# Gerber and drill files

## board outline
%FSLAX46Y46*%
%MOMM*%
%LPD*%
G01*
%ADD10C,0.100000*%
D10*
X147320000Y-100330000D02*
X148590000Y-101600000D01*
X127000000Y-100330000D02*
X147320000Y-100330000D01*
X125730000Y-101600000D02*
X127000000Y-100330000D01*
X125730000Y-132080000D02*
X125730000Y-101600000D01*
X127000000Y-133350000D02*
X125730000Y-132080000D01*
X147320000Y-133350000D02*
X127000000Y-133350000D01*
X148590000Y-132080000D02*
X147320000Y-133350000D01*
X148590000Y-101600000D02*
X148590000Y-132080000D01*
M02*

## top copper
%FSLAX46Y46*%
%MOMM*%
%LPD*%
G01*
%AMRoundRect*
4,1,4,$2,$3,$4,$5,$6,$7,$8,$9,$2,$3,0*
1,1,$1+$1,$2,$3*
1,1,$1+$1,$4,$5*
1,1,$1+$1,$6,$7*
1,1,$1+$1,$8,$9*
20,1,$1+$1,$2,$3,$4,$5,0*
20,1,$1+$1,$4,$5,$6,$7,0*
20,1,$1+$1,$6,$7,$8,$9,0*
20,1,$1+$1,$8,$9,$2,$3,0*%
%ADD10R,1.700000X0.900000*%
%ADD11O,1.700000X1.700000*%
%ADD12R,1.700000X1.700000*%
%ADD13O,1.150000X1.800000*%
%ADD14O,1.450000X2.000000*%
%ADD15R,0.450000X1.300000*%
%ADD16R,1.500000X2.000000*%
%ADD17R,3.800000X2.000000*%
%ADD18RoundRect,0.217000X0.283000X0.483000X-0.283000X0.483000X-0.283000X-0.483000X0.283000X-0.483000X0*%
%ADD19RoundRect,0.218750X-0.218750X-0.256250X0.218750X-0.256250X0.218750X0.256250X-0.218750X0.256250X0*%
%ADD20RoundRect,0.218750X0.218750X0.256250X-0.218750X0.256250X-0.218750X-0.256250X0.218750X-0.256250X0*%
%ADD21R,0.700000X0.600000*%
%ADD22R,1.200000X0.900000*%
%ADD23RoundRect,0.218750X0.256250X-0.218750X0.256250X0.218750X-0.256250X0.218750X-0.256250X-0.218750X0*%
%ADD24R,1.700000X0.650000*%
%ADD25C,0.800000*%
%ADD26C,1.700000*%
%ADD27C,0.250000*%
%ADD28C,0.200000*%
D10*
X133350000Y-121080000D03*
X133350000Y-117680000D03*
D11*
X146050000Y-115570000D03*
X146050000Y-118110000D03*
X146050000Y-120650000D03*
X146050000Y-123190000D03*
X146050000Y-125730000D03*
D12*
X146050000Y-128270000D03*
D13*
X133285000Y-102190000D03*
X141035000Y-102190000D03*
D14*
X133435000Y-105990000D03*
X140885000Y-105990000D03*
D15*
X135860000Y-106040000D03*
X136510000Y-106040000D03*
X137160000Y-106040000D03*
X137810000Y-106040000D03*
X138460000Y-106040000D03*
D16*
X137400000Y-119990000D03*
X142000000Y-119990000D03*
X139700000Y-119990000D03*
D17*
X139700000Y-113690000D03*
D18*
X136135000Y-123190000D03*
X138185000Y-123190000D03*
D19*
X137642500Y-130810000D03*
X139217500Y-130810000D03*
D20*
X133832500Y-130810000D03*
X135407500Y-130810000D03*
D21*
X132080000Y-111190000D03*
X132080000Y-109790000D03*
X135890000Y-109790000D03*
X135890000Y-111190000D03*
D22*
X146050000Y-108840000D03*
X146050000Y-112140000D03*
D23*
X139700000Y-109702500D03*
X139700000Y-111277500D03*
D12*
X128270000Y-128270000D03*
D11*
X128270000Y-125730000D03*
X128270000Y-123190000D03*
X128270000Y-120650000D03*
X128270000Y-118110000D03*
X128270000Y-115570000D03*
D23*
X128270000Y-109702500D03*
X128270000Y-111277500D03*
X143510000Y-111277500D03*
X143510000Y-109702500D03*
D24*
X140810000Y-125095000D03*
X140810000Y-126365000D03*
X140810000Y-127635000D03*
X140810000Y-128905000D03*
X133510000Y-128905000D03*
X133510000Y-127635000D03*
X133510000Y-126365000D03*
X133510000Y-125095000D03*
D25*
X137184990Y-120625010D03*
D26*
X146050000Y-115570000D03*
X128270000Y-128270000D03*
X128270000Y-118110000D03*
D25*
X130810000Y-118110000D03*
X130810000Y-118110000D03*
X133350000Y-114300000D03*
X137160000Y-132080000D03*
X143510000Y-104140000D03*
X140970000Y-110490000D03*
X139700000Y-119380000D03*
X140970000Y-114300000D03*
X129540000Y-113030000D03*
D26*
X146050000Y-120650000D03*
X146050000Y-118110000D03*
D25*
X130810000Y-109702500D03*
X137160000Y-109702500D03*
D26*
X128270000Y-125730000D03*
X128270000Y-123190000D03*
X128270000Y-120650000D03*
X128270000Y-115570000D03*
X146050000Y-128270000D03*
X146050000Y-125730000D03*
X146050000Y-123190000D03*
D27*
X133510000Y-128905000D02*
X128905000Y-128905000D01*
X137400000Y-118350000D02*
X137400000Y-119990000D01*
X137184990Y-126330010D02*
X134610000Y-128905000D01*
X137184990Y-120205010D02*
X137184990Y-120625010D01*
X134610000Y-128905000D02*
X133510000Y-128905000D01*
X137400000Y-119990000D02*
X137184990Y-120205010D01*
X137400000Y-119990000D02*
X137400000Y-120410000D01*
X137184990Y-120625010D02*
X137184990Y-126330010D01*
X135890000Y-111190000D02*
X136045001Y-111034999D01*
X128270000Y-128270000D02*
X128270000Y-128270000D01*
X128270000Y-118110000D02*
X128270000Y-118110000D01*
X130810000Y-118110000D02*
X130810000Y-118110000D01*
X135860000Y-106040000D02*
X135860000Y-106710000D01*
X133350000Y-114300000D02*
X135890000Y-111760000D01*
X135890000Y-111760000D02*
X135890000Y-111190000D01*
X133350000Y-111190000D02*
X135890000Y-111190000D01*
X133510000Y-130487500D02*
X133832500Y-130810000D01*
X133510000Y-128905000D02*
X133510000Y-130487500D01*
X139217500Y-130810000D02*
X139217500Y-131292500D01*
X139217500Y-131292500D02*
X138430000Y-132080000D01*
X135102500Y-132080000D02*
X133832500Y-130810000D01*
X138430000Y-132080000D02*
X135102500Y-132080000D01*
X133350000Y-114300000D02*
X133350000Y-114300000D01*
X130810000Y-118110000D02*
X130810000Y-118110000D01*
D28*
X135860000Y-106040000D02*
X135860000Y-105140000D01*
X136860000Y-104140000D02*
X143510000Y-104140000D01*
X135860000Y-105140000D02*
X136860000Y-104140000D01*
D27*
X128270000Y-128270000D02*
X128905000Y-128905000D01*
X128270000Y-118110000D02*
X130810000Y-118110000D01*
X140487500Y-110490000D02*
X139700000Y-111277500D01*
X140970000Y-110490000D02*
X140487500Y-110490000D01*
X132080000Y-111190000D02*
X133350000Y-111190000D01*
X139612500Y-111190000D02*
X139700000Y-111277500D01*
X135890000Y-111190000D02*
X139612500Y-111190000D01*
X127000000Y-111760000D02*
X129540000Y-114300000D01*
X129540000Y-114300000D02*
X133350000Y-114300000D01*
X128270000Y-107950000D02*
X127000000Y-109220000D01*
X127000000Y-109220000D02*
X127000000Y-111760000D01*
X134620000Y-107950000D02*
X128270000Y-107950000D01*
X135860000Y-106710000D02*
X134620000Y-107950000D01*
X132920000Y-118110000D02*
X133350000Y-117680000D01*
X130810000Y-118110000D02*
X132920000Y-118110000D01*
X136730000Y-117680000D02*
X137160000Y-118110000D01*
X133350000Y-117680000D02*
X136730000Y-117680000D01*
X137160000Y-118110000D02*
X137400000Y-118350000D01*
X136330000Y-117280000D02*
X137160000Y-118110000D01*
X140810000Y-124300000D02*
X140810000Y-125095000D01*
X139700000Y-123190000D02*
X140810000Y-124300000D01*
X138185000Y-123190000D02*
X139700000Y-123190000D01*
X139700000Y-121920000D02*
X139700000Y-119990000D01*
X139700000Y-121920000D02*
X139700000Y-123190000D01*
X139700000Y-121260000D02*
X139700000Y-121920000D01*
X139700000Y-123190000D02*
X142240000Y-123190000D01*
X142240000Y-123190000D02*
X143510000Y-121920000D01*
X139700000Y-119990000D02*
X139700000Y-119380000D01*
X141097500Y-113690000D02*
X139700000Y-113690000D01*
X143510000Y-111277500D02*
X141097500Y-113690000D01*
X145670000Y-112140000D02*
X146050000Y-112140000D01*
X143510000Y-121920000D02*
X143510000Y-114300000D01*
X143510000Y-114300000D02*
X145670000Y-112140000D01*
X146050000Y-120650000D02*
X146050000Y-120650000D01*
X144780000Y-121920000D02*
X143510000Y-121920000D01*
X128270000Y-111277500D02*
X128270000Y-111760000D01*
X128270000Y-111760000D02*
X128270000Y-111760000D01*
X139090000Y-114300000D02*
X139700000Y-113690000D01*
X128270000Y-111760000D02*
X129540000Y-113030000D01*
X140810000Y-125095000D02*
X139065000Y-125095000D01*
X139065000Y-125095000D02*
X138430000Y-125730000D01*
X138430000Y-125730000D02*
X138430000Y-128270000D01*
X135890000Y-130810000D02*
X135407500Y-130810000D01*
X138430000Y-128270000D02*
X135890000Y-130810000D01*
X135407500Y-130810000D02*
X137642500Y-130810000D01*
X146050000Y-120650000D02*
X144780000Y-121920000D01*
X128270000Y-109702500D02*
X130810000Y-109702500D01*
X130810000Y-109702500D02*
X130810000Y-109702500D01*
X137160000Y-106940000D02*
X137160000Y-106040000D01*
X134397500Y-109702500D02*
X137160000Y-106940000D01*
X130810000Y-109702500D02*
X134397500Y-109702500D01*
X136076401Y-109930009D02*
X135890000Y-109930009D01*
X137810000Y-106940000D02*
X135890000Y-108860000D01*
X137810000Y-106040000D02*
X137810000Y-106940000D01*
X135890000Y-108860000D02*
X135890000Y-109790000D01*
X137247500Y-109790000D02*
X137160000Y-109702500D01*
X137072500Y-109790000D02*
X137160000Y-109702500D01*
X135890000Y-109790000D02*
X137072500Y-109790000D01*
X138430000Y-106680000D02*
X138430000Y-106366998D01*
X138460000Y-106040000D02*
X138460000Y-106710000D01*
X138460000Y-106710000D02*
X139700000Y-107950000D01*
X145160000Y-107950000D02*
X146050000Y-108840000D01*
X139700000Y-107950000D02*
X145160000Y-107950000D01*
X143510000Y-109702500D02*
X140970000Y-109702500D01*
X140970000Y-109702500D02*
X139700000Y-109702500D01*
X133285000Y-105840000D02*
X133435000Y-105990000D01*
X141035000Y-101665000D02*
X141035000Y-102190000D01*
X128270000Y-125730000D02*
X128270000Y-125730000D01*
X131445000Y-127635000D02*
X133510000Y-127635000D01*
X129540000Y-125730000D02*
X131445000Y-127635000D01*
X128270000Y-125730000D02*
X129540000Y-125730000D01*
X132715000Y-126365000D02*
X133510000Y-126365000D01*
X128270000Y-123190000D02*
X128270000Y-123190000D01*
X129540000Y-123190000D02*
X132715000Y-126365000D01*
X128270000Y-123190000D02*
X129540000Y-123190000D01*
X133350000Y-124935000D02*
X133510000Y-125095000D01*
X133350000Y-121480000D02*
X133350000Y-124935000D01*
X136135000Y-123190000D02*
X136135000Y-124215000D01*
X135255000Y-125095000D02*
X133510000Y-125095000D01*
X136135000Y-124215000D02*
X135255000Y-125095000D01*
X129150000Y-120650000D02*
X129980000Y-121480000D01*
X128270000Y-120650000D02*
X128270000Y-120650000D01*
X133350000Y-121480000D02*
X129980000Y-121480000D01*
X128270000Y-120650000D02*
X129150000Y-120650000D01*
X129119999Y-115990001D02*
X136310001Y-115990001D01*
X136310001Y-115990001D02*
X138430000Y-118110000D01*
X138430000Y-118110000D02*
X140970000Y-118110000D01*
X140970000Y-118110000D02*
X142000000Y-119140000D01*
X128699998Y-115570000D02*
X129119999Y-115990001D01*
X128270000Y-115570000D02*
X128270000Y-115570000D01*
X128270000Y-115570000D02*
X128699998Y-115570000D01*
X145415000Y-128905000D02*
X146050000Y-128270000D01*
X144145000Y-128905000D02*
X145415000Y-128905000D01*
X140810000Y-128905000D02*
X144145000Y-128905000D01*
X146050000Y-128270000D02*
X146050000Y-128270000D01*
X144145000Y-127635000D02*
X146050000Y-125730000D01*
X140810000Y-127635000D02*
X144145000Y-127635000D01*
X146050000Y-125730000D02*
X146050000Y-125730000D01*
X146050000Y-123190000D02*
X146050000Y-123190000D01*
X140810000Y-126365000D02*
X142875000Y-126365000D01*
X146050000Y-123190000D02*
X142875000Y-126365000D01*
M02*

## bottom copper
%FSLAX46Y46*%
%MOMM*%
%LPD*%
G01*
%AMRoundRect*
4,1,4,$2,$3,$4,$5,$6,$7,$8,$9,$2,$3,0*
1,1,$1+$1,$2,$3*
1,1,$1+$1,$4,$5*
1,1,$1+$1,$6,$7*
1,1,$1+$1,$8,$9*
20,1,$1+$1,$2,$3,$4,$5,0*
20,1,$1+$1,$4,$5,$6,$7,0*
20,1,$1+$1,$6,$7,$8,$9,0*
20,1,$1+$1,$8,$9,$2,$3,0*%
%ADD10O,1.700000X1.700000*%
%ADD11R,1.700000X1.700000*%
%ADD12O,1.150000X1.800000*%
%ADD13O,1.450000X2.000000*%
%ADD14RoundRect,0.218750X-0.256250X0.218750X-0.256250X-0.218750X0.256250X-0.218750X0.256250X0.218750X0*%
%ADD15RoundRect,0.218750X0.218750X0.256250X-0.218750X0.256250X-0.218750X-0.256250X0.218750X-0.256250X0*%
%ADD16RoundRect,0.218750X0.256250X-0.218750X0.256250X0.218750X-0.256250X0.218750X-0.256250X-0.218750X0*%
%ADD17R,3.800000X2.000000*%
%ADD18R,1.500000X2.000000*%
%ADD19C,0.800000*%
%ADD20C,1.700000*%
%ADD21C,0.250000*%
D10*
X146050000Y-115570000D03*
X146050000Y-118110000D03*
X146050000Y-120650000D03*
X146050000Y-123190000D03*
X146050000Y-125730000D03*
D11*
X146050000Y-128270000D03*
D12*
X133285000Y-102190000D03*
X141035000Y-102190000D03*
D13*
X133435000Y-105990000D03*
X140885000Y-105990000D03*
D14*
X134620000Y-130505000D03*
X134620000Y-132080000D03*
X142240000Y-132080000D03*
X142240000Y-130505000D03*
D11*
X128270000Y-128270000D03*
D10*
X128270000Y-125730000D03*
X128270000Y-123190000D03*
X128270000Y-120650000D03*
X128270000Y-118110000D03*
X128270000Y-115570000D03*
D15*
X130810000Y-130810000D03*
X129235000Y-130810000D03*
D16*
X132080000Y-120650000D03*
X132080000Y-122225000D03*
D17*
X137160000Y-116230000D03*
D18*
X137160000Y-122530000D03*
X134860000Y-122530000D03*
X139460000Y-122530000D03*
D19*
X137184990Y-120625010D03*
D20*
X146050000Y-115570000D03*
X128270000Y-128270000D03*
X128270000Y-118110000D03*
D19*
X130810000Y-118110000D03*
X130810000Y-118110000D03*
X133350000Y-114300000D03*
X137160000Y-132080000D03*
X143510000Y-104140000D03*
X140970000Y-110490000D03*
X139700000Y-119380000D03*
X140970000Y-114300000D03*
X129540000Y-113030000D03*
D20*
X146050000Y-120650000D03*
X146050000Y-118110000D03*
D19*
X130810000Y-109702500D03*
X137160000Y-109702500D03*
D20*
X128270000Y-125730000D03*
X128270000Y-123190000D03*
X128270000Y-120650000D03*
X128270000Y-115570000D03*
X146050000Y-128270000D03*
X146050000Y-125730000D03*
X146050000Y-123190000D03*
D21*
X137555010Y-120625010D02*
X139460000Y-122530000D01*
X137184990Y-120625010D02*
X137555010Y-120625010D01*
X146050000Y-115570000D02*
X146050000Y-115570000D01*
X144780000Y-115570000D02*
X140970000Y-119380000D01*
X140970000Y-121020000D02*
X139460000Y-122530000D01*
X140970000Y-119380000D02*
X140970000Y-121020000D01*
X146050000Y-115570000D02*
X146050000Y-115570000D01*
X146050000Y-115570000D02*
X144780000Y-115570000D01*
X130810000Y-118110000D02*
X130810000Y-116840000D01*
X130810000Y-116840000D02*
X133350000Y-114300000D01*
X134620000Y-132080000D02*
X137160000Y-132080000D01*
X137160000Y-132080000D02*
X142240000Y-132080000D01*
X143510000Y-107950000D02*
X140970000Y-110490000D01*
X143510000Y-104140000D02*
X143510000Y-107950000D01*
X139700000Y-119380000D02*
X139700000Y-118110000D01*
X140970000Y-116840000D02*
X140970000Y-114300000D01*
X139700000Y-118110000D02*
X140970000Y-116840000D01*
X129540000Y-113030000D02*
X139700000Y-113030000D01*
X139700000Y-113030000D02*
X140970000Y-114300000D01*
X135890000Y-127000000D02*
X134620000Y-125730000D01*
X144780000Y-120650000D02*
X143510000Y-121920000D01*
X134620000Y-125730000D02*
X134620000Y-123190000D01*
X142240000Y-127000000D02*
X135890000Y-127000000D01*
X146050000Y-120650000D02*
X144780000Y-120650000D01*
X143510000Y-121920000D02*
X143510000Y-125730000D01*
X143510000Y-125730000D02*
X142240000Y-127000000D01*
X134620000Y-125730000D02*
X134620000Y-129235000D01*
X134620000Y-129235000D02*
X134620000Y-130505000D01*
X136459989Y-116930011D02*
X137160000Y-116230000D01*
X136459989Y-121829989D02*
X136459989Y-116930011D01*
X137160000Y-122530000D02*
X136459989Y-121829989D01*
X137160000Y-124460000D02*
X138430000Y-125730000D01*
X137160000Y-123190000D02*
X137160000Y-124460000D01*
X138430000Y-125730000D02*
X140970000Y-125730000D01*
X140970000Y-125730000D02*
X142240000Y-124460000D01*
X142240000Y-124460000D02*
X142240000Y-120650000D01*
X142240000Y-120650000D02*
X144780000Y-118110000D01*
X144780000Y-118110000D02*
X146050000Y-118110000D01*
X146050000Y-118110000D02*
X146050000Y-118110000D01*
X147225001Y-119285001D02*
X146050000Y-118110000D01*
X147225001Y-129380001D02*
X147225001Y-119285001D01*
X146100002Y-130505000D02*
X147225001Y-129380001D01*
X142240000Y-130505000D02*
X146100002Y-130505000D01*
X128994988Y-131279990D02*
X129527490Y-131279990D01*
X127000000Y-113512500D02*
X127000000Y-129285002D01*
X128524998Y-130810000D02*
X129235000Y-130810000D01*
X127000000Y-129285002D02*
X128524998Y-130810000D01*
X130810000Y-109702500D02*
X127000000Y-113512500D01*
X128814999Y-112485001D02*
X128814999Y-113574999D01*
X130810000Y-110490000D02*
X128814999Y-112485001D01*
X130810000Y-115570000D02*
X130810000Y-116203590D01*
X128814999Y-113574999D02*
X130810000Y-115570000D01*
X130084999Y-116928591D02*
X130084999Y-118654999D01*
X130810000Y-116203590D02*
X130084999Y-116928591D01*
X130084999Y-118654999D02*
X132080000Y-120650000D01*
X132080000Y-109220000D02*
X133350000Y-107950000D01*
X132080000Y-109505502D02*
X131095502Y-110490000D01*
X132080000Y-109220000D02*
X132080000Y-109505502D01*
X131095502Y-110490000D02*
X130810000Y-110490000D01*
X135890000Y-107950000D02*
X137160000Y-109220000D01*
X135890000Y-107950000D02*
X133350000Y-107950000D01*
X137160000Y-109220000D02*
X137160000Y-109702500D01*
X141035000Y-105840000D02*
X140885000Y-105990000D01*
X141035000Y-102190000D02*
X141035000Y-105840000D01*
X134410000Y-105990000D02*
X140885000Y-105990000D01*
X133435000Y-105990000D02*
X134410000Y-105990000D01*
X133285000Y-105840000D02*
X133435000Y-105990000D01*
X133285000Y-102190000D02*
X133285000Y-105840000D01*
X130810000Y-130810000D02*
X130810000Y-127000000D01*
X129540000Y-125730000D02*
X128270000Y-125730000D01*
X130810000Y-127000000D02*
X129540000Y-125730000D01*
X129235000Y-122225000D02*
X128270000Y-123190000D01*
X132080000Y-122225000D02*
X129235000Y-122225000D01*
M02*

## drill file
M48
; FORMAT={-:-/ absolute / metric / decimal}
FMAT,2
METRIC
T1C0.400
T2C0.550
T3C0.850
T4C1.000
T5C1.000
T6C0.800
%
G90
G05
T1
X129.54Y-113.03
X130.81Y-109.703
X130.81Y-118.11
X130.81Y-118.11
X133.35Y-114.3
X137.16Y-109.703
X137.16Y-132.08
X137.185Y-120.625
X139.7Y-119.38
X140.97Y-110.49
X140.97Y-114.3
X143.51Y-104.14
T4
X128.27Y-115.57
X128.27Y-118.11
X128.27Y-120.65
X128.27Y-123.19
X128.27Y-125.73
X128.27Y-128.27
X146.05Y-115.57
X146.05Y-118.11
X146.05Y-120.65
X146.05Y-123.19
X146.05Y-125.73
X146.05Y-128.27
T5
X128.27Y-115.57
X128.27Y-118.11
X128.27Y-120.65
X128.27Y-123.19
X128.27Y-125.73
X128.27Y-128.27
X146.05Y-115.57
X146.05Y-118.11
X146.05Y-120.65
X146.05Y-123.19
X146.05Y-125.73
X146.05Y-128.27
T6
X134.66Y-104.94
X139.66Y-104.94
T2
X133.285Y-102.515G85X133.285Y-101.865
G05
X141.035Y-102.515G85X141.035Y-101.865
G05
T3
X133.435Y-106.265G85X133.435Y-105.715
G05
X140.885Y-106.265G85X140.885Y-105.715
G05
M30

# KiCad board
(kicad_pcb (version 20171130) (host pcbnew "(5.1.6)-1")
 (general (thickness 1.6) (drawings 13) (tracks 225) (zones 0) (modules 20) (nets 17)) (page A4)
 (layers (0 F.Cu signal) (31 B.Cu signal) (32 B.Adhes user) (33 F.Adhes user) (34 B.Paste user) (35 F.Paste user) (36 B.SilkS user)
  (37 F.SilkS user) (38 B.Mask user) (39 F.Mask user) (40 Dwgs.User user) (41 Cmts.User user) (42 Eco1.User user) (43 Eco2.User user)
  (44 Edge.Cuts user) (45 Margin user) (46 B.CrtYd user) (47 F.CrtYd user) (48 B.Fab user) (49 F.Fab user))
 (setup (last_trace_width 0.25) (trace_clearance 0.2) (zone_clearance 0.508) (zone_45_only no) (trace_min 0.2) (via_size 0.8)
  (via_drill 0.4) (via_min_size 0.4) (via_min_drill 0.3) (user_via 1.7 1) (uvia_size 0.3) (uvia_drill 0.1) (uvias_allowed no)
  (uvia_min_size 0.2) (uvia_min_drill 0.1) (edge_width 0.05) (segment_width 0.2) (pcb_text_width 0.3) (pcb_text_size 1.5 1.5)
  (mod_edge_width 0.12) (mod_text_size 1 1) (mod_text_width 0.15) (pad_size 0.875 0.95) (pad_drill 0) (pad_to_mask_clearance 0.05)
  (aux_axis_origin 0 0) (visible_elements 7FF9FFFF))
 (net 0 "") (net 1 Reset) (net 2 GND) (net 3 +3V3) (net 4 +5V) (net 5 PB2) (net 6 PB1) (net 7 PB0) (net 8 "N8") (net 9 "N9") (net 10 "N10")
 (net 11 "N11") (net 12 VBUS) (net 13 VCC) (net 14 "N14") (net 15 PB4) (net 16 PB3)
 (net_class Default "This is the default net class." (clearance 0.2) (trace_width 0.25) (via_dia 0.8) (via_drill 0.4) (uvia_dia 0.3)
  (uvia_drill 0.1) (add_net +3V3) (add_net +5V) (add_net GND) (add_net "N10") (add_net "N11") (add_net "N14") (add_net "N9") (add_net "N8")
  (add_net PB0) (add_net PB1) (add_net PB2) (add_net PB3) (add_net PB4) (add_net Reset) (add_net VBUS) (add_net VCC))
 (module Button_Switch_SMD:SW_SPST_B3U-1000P (layer F.Cu) (at 133.35 119.38 270)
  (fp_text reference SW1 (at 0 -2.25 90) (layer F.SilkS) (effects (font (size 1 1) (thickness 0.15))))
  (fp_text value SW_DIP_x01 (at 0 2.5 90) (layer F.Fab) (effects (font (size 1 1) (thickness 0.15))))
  (pad 2 smd rect (at 1.7 0 270) (size 0.9 1.7) (layers F.Cu F.Paste F.Mask) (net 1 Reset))
  (pad 1 smd rect (at -1.7 0 270) (size 0.9 1.7) (layers F.Cu F.Paste F.Mask) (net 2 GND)))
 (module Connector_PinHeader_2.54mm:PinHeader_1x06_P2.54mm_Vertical (layer B.Cu) (at 146.05 128.27)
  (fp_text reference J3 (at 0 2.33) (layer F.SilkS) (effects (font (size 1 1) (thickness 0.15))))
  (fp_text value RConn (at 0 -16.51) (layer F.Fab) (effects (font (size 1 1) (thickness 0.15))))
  (pad 6 thru_hole oval (at 0 -12.7) (size 1.7 1.7) (drill 1) (layers *.Cu *.Mask) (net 2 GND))
  (pad 5 thru_hole oval (at 0 -10.16) (size 1.7 1.7) (drill 1) (layers *.Cu *.Mask) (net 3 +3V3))
  (pad 4 thru_hole oval (at 0 -7.62) (size 1.7 1.7) (drill 1) (layers *.Cu *.Mask) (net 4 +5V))
  (pad 3 thru_hole oval (at 0 -5.08) (size 1.7 1.7) (drill 1) (layers *.Cu *.Mask) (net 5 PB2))
  (pad 2 thru_hole oval (at 0 -2.54) (size 1.7 1.7) (drill 1) (layers *.Cu *.Mask) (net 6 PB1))
  (pad 1 thru_hole rect (at 0 0) (size 1.7 1.7) (drill 1) (layers *.Cu *.Mask) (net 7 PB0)))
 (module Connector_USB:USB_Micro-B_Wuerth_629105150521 (layer F.Cu) (at 137.16 104.14 180)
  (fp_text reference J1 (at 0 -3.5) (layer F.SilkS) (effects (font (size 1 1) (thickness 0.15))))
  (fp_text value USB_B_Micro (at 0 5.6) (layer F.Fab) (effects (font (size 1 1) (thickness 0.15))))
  (pad "" np_thru_hole oval (at 2.5 -0.8 180) (size 0.8 0.8) (drill 0.8) (layers *.Cu *.Mask))
  (pad "" np_thru_hole oval (at -2.5 -0.8 180) (size 0.8 0.8) (drill 0.8) (layers *.Cu *.Mask))
  (pad 6 thru_hole oval (at 3.875 1.95 180) (size 1.15 1.8) (drill oval 0.55 1.2) (layers *.Cu *.Mask) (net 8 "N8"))
  (pad 6 thru_hole oval (at -3.875 1.95 180) (size 1.15 1.8) (drill oval 0.55 1.2) (layers *.Cu *.Mask) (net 8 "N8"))
  (pad 6 thru_hole oval (at 3.725 -1.85 180) (size 1.45 2) (drill oval 0.85 1.4) (layers *.Cu *.Mask) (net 8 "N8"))
  (pad 6 thru_hole oval (at -3.725 -1.85 180) (size 1.45 2) (drill oval 0.85 1.4) (layers *.Cu *.Mask) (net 8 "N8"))
  (pad 5 smd rect (at 1.3 -1.9 180) (size 0.45 1.3) (layers F.Cu F.Paste F.Mask) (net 2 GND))
  (pad 4 smd rect (at 0.65 -1.9 180) (size 0.45 1.3) (layers F.Cu F.Paste F.Mask) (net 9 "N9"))
  (pad 3 smd rect (at 0 -1.9 180) (size 0.45 1.3) (layers F.Cu F.Paste F.Mask) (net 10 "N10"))
  (pad 2 smd rect (at -0.65 -1.9 180) (size 0.45 1.3) (layers F.Cu F.Paste F.Mask) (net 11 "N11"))
  (pad 1 smd rect (at -1.3 -1.9 180) (size 0.45 1.3) (layers F.Cu F.Paste F.Mask) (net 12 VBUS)))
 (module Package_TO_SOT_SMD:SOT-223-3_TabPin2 (layer F.Cu) (at 139.7 116.84 90)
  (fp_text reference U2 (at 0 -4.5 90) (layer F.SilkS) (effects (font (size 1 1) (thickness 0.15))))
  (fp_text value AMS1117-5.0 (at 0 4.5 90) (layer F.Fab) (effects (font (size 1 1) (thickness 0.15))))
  (pad 1 smd rect (at -3.15 -2.3 90) (size 2 1.5) (layers F.Cu F.Paste F.Mask) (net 2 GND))
  (pad 3 smd rect (at -3.15 2.3 90) (size 2 1.5) (layers F.Cu F.Paste F.Mask) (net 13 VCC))
  (pad 2 smd rect (at -3.15 0 90) (size 2 1.5) (layers F.Cu F.Paste F.Mask) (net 4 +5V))
  (pad 2 smd rect (at 3.15 0 90) (size 2 3.8) (layers F.Cu F.Paste F.Mask) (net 4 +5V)))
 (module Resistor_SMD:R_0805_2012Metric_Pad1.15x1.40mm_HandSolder (layer F.Cu) (at 137.16 123.19 180)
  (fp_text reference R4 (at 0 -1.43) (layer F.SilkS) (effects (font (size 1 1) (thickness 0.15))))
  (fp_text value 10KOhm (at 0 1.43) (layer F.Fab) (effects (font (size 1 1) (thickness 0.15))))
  (pad 2 smd roundrect (at 1.025 0 180) (size 1 1.4) (layers F.Cu F.Paste F.Mask) (roundrect_rratio 0.217) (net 1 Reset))
  (pad 1 smd roundrect (at -1.025 0 180) (size 1 1.4) (layers F.Cu F.Paste F.Mask) (roundrect_rratio 0.217) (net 4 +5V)))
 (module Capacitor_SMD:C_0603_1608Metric (layer F.Cu) (at 138.43 130.81)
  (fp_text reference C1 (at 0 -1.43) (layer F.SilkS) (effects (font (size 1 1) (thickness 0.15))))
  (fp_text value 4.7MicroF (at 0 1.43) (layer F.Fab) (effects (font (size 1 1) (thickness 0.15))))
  (pad 1 smd roundrect (at -0.7875 0) (size 0.875 0.95) (layers F.Cu F.Paste F.Mask) (roundrect_rratio 0.25) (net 4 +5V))
  (pad 2 smd roundrect (at 0.7875 0) (size 0.875 0.95) (layers F.Cu F.Paste F.Mask) (roundrect_rratio 0.25) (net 2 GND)))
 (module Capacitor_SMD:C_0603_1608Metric (layer F.Cu) (at 134.62 130.81 180)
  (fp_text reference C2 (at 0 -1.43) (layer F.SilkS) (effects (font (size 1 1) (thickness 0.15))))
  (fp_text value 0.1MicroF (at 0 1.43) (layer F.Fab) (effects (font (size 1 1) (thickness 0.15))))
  (pad 2 smd roundrect (at 0.7875 0 180) (size 0.875 0.95) (layers F.Cu F.Paste F.Mask) (roundrect_rratio 0.25) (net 2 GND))
  (pad 1 smd roundrect (at -0.7875 0 180) (size 0.875 0.95) (layers F.Cu F.Paste F.Mask) (roundrect_rratio 0.25) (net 4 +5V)))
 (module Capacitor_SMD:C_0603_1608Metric (layer B.Cu) (at 134.62 131.2925 270)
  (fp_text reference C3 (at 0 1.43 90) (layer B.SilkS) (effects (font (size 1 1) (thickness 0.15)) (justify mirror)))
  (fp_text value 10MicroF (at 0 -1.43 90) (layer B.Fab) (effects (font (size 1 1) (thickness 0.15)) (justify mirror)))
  (pad 1 smd roundrect (at -0.7875 0 270) (size 0.875 0.95) (layers B.Cu B.Paste B.Mask) (roundrect_rratio 0.25) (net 4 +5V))
  (pad 2 smd roundrect (at 0.7875 0 270) (size 0.875 0.95) (layers B.Cu B.Paste B.Mask) (roundrect_rratio 0.25) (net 2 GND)))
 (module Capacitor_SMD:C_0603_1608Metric (layer B.Cu) (at 142.24 131.2925 270)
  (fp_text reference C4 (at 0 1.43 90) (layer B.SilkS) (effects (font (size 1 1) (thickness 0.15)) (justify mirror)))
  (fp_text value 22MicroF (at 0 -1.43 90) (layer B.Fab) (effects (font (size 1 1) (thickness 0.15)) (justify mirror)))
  (pad 2 smd roundrect (at 0.7875 0 270) (size 0.875 0.95) (layers B.Cu B.Paste B.Mask) (roundrect_rratio 0.25) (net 2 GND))
  (pad 1 smd roundrect (at -0.7875 0 270) (size 0.875 0.95) (layers B.Cu B.Paste B.Mask) (roundrect_rratio 0.25) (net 3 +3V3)))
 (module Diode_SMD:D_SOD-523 (layer F.Cu) (at 132.08 110.49 270)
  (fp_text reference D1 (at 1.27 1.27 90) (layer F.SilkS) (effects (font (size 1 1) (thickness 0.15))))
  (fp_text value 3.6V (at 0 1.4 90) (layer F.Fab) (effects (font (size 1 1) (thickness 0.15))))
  (pad 2 smd rect (at 0.7 0 90) (size 0.6 0.7) (layers F.Cu F.Paste F.Mask) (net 2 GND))
  (pad 1 smd rect (at -0.7 0 90) (size 0.6 0.7) (layers F.Cu F.Paste F.Mask) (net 10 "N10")))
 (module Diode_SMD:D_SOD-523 (layer F.Cu) (at 135.89 110.49 270)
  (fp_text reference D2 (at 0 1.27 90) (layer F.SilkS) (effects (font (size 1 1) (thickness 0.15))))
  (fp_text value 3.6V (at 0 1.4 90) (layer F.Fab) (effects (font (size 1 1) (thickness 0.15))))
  (pad 1 smd rect (at -0.7 0 90) (size 0.6 0.7) (layers F.Cu F.Paste F.Mask) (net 11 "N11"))
  (pad 2 smd rect (at 0.7 0 90) (size 0.6 0.7) (layers F.Cu F.Paste F.Mask) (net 2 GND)))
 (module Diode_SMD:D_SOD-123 (layer F.Cu) (at 146.05 110.49 90)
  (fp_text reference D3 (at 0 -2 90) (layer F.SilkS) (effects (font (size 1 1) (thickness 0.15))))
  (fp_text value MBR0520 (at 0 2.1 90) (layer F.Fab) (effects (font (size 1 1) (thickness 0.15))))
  (pad 2 smd rect (at 1.65 0 90) (size 0.9 1.2) (layers F.Cu F.Paste F.Mask) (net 12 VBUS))
  (pad 1 smd rect (at -1.65 0 90) (size 0.9 1.2) (layers F.Cu F.Paste F.Mask) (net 4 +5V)))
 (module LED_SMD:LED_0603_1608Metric (layer F.Cu) (at 139.7 110.49 90)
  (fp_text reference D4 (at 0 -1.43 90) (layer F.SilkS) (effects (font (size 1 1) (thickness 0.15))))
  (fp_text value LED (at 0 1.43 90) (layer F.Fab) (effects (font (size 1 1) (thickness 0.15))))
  (pad 2 smd roundrect (at 0.7875 0 90) (size 0.875 0.95) (layers F.Cu F.Paste F.Mask) (roundrect_rratio 0.25) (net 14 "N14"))
  (pad 1 smd roundrect (at -0.7875 0 90) (size 0.875 0.95) (layers F.Cu F.Paste F.Mask) (roundrect_rratio 0.25) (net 2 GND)))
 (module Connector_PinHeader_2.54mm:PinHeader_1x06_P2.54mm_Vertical (layer B.Cu) (at 128.27 128.27)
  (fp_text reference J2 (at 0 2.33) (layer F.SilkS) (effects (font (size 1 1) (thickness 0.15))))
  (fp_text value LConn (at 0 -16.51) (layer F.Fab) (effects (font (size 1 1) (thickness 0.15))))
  (pad 1 thru_hole rect (at 0 0) (size 1.7 1.7) (drill 1) (layers *.Cu *.Mask) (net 2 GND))
  (pad 2 thru_hole oval (at 0 -2.54) (size 1.7 1.7) (drill 1) (layers *.Cu *.Mask) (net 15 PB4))
  (pad 3 thru_hole oval (at 0 -5.08) (size 1.7 1.7) (drill 1) (layers *.Cu *.Mask) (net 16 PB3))
  (pad 4 thru_hole oval (at 0 -7.62) (size 1.7 1.7) (drill 1) (layers *.Cu *.Mask) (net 1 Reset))
  (pad 5 thru_hole oval (at 0 -10.16) (size 1.7 1.7) (drill 1) (layers *.Cu *.Mask) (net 2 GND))
  (pad 6 thru_hole oval (at 0 -12.7) (size 1.7 1.7) (drill 1) (layers *.Cu *.Mask) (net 13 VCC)))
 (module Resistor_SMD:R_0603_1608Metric (layer F.Cu) (at 128.27 110.49 90)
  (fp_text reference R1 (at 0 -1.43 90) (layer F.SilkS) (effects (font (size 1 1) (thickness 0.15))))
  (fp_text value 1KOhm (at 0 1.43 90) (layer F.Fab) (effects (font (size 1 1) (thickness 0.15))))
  (pad 2 smd roundrect (at 0.7875 0 90) (size 0.875 0.95) (layers F.Cu F.Paste F.Mask) (roundrect_rratio 0.25) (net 10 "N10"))
  (pad 1 smd roundrect (at -0.7875 0 90) (size 0.875 0.95) (layers F.Cu F.Paste F.Mask) (roundrect_rratio 0.25) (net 4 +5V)))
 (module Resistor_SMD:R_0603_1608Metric (layer B.Cu) (at 130.0225 130.81 180)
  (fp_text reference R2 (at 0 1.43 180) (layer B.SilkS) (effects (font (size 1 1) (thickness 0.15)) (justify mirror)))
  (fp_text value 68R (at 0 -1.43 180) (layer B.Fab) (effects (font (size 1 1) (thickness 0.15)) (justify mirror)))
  (pad 1 smd roundrect (at -0.7875 0 180) (size 0.875 0.95) (layers B.Cu B.Paste B.Mask) (roundrect_rratio 0.25) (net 15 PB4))
  (pad 2 smd roundrect (at 0.7875 0 180) (size 0.875 0.95) (layers B.Cu B.Paste B.Mask) (roundrect_rratio 0.25) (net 10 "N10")))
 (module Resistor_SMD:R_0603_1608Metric (layer B.Cu) (at 132.08 121.4375 90)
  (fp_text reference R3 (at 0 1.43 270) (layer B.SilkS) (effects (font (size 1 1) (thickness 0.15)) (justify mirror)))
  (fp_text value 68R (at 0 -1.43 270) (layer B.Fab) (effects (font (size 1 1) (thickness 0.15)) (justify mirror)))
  (pad 2 smd roundrect (at 0.7875 0 90) (size 0.875 0.95) (layers B.Cu B.Paste B.Mask) (roundrect_rratio 0.25) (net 11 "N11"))
  (pad 1 smd roundrect (at -0.7875 0 90) (size 0.875 0.95) (layers B.Cu B.Paste B.Mask) (roundrect_rratio 0.25) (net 16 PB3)))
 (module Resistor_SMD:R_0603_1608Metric (layer F.Cu) (at 143.51 110.49 90)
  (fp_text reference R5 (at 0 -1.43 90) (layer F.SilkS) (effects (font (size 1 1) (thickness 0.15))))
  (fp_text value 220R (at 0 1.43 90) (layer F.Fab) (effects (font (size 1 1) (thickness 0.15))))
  (pad 1 smd roundrect (at -0.7875 0 90) (size 0.875 0.95) (layers F.Cu F.Paste F.Mask) (roundrect_rratio 0.25) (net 4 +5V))
  (pad 2 smd roundrect (at 0.7875 0 90) (size 0.875 0.95) (layers F.Cu F.Paste F.Mask) (roundrect_rratio 0.25) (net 14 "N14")))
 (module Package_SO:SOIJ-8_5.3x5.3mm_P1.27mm (layer F.Cu) (at 137.16 127)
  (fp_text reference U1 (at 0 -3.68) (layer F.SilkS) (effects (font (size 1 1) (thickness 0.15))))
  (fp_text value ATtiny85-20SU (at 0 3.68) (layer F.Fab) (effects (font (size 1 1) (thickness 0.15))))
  (pad 8 smd rect (at 3.65 -1.905) (size 1.7 0.65) (layers F.Cu F.Paste F.Mask) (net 4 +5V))
  (pad 7 smd rect (at 3.65 -0.635) (size 1.7 0.65) (layers F.Cu F.Paste F.Mask) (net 5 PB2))
  (pad 6 smd rect (at 3.65 0.635) (size 1.7 0.65) (layers F.Cu F.Paste F.Mask) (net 6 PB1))
  (pad 5 smd rect (at 3.65 1.905) (size 1.7 0.65) (layers F.Cu F.Paste F.Mask) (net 7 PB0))
  (pad 4 smd rect (at -3.65 1.905) (size 1.7 0.65) (layers F.Cu F.Paste F.Mask) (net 2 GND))
  (pad 3 smd rect (at -3.65 0.635) (size 1.7 0.65) (layers F.Cu F.Paste F.Mask) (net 15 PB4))
  (pad 2 smd rect (at -3.65 -0.635) (size 1.7 0.65) (layers F.Cu F.Paste F.Mask) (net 16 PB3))
  (pad 1 smd rect (at -3.65 -1.905) (size 1.7 0.65) (layers F.Cu F.Paste F.Mask) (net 1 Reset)))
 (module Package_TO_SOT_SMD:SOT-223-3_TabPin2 (layer B.Cu) (at 137.16 119.38 90)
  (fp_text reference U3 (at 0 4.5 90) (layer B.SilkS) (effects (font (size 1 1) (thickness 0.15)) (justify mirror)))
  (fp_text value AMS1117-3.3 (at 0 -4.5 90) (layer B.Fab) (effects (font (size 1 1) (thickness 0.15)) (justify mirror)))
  (pad 2 smd rect (at 3.15 0 90) (size 2 3.8) (layers B.Cu B.Paste B.Mask) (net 3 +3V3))
  (pad 2 smd rect (at -3.15 0 90) (size 2 1.5) (layers B.Cu B.Paste B.Mask) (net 3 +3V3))
  (pad 3 smd rect (at -3.15 -2.3 90) (size 2 1.5) (layers B.Cu B.Paste B.Mask) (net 4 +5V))
  (pad 1 smd rect (at -3.15 2.3 90) (size 2 1.5) (layers B.Cu B.Paste B.Mask) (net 2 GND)))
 (gr_line (start 147.32 100.33) (end 148.59 101.6) (layer Edge.Cuts) (width 0.1))
 (gr_line (start 127 100.33) (end 147.32 100.33) (layer Edge.Cuts) (width 0.1))
 (gr_line (start 125.73 101.6) (end 127 100.33) (layer Edge.Cuts) (width 0.1))
 (gr_line (start 125.73 132.08) (end 125.73 101.6) (layer Edge.Cuts) (width 0.1))
 (gr_line (start 127 133.35) (end 125.73 132.08) (layer Edge.Cuts) (width 0.1))
 (gr_line (start 147.32 133.35) (end 127 133.35) (layer Edge.Cuts) (width 0.1))
 (gr_line (start 148.59 132.08) (end 147.32 133.35) (layer Edge.Cuts) (width 0.1))
 (gr_line (start 148.59 101.6) (end 148.59 132.08) (layer Edge.Cuts) (width 0.1))
 (segment (start 133.51 128.905) (end 128.905 128.905) (width 0.25) (layer F.Cu) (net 2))
 (segment (start 137.4 118.35) (end 137.4 119.99) (width 0.25) (layer F.Cu) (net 2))
 (segment (start 137.18499 126.33001) (end 134.61 128.905) (width 0.25) (layer F.Cu) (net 2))
 (segment (start 137.18499 120.20501) (end 137.18499 120.62501) (width 0.25) (layer F.Cu) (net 2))
 (segment (start 134.61 128.905) (end 133.51 128.905) (width 0.25) (layer F.Cu) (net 2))
 (segment (start 137.4 119.99) (end 137.18499 120.20501) (width 0.25) (layer F.Cu) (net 2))
 (segment (start 137.4 119.99) (end 137.4 120.41) (width 0.25) (layer F.Cu) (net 2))
 (segment (start 137.18499 120.62501) (end 137.18499 126.33001) (width 0.25) (layer F.Cu) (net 2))
 (via (at 137.18499 120.62501) (size 0.8) (drill 0.4) (layers F.Cu B.Cu) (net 2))
 (segment (start 137.55501 120.62501) (end 139.46 122.53) (width 0.25) (layer B.Cu) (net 2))
 (segment (start 137.18499 120.62501) (end 137.55501 120.62501) (width 0.25) (layer B.Cu) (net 2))
 (segment (start 135.89 111.19) (end 136.045001 111.034999) (width 0.25) (layer F.Cu) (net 2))
 (segment (start 128.27 128.27) (end 128.27 128.27) (width 0.25) (layer F.Cu) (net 2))
 (segment (start 128.27 118.11) (end 128.27 118.11) (width 0.25) (layer F.Cu) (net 2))
 (segment (start 130.81 118.11) (end 130.81 118.11) (width 0.25) (layer F.Cu) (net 2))
 (segment (start 135.86 106.04) (end 135.86 106.71) (width 0.25) (layer F.Cu) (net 2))
 (segment (start 133.35 114.3) (end 135.89 111.76) (width 0.25) (layer F.Cu) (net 2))
 (segment (start 135.89 111.76) (end 135.89 111.19) (width 0.25) (layer F.Cu) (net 2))
 (segment (start 133.35 111.19) (end 135.89 111.19) (width 0.25) (layer F.Cu) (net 2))
 (segment (start 133.51 130.4875) (end 133.8325 130.81) (width 0.25) (layer F.Cu) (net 2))
 (segment (start 133.51 128.905) (end 133.51 130.4875) (width 0.25) (layer F.Cu) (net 2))
 (segment (start 139.2175 130.81) (end 139.2175 131.2925) (width 0.25) (layer F.Cu) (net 2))
 (segment (start 139.2175 131.2925) (end 138.43 132.08) (width 0.25) (layer F.Cu) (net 2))
 (segment (start 135.1025 132.08) (end 133.8325 130.81) (width 0.25) (layer F.Cu) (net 2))
 (segment (start 138.43 132.08) (end 135.1025 132.08) (width 0.25) (layer F.Cu) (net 2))
 (segment (start 133.35 114.3) (end 133.35 114.3) (width 0.25) (layer F.Cu) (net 2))
 (segment (start 130.81 118.11) (end 130.81 118.11) (width 0.25) (layer F.Cu) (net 2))
 (segment (start 146.05 115.57) (end 146.05 115.57) (width 0.25) (layer B.Cu) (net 2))
 (segment (start 144.78 115.57) (end 140.97 119.38) (width 0.25) (layer B.Cu) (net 2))
 (segment (start 140.97 121.02) (end 139.46 122.53) (width 0.25) (layer B.Cu) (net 2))
 (segment (start 140.97 119.38) (end 140.97 121.02) (width 0.25) (layer B.Cu) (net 2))
 (segment (start 135.86 106.04) (end 135.86 105.14) (width 0.2) (layer F.Cu) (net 2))
 (segment (start 136.86 104.14) (end 143.51 104.14) (width 0.2) (layer F.Cu) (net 2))
 (segment (start 135.86 105.14) (end 136.86 104.14) (width 0.2) (layer F.Cu) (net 2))
 (segment (start 146.05 115.57) (end 146.05 115.57) (width 0.25) (layer B.Cu) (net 2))
 (segment (start 146.05 115.57) (end 144.78 115.57) (width 0.25) (layer B.Cu) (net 2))
 (via (at 146.05 115.57) (size 1.7) (drill 1) (layers F.Cu B.Cu) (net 2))
 (segment (start 128.27 128.27) (end 128.905 128.905) (width 0.25) (layer F.Cu) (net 2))
 (via (at 128.27 128.27) (size 1.7) (drill 1) (layers F.Cu B.Cu) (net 2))
 (segment (start 128.27 118.11) (end 130.81 118.11) (width 0.25) (layer F.Cu) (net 2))
 (via (at 128.27 118.11) (size 1.7) (drill 1) (layers F.Cu B.Cu) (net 2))
 (segment (start 130.81 118.11) (end 130.81 116.84) (width 0.25) (layer B.Cu) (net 2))
 (via (at 130.81 118.11) (size 0.8) (drill 0.4) (layers F.Cu B.Cu) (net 2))
 (via (at 130.81 118.11) (size 0.8) (drill 0.4) (layers F.Cu B.Cu) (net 2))
 (segment (start 130.81 116.84) (end 133.35 114.3) (width 0.25) (layer B.Cu) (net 2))
 (via (at 133.35 114.3) (size 0.8) (drill 0.4) (layers F.Cu B.Cu) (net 2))
 (segment (start 134.62 132.08) (end 137.16 132.08) (width 0.25) (layer B.Cu) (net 2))
 (segment (start 137.16 132.08) (end 142.24 132.08) (width 0.25) (layer B.Cu) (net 2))
 (via (at 137.16 132.08) (size 0.8) (drill 0.4) (layers F.Cu B.Cu) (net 2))
 (segment (start 140.4875 110.49) (end 139.7 111.2775) (width 0.25) (layer F.Cu) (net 2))
 (via (at 143.51 104.14) (size 0.8) (drill 0.4) (layers F.Cu B.Cu) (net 2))
 (segment (start 140.97 110.49) (end 140.4875 110.49) (width 0.25) (layer F.Cu) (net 2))
 (via (at 140.97 110.49) (size 0.8) (drill 0.4) (layers F.Cu B.Cu) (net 2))
 (segment (start 143.51 107.95) (end 140.97 110.49) (width 0.25) (layer B.Cu) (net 2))
 (segment (start 143.51 104.14) (end 143.51 107.95) (width 0.25) (layer B.Cu) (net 2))
 (segment (start 132.08 111.19) (end 133.35 111.19) (width 0.25) (layer F.Cu) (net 2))
 (segment (start 139.6125 111.19) (end 139.7 111.2775) (width 0.25) (layer F.Cu) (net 2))
 (segment (start 135.89 111.19) (end 139.6125 111.19) (width 0.25) (layer F.Cu) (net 2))
 (segment (start 127 111.76) (end 129.54 114.3) (width 0.25) (layer F.Cu) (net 2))
 (segment (start 129.54 114.3) (end 133.35 114.3) (width 0.25) (layer F.Cu) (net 2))
 (segment (start 128.27 107.95) (end 127 109.22) (width 0.25) (layer F.Cu) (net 2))
 (segment (start 127 109.22) (end 127 111.76) (width 0.25) (layer F.Cu) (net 2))
 (segment (start 134.62 107.95) (end 128.27 107.95) (width 0.25) (layer F.Cu) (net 2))
 (segment (start 135.86 106.71) (end 134.62 107.95) (width 0.25) (layer F.Cu) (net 2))
 (segment (start 132.92 118.11) (end 133.35 117.68) (width 0.25) (layer F.Cu) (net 2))
 (segment (start 130.81 118.11) (end 132.92 118.11) (width 0.25) (layer F.Cu) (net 2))
 (segment (start 136.73 117.68) (end 137.16 118.11) (width 0.25) (layer F.Cu) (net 2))
 (segment (start 133.35 117.68) (end 136.73 117.68) (width 0.25) (layer F.Cu) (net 2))
 (segment (start 137.16 118.11) (end 137.4 118.35) (width 0.25) (layer F.Cu) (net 2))
 (segment (start 136.33 117.28) (end 137.16 118.11) (width 0.25) (layer F.Cu) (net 2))
 (via (at 139.7 119.38) (size 0.8) (drill 0.4) (layers F.Cu B.Cu) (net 4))
 (via (at 140.97 114.3) (size 0.8) (drill 0.4) (layers F.Cu B.Cu) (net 4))
 (segment (start 140.81 124.3) (end 140.81 125.095) (width 0.25) (layer F.Cu) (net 4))
 (segment (start 139.7 123.19) (end 140.81 124.3) (width 0.25) (layer F.Cu) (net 4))
 (segment (start 138.185 123.19) (end 139.7 123.19) (width 0.25) (layer F.Cu) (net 4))
 (segment (start 139.7 121.92) (end 139.7 119.99) (width 0.25) (layer F.Cu) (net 4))
 (segment (start 139.7 121.92) (end 139.7 123.19) (width 0.25) (layer F.Cu) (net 4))
 (segment (start 139.7 121.26) (end 139.7 121.92) (width 0.25) (layer F.Cu) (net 4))
 (segment (start 139.7 123.19) (end 142.24 123.19) (width 0.25) (layer F.Cu) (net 4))
 (segment (start 142.24 123.19) (end 143.51 121.92) (width 0.25) (layer F.Cu) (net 4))
 (segment (start 139.7 119.99) (end 139.7 119.38) (width 0.25) (layer F.Cu) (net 4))
 (segment (start 139.7 119.38) (end 139.7 118.11) (width 0.25) (layer B.Cu) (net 4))
 (segment (start 140.97 116.84) (end 140.97 114.3) (width 0.25) (layer B.Cu) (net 4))
 (segment (start 139.7 118.11) (end 140.97 116.84) (width 0.25) (layer B.Cu) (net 4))
 (segment (start 141.0975 113.69) (end 139.7 113.69) (width 0.25) (layer F.Cu) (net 4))
 (segment (start 143.51 111.2775) (end 141.0975 113.69) (width 0.25) (layer F.Cu) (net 4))
 (segment (start 145.67 112.14) (end 146.05 112.14) (width 0.25) (layer F.Cu) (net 4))
 (segment (start 143.51 121.92) (end 143.51 114.3) (width 0.25) (layer F.Cu) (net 4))
 (segment (start 143.51 114.3) (end 145.67 112.14) (width 0.25) (layer F.Cu) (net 4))
 (segment (start 146.05 120.65) (end 146.05 120.65) (width 0.25) (layer F.Cu) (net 4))
 (segment (start 144.78 121.92) (end 143.51 121.92) (width 0.25) (layer F.Cu) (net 4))
 (segment (start 128.27 111.2775) (end 128.27 111.76) (width 0.25) (layer F.Cu) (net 4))
 (segment (start 128.27 111.76) (end 128.27 111.76) (width 0.25) (layer F.Cu) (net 4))
 (segment (start 139.09 114.3) (end 139.7 113.69) (width 0.25) (layer F.Cu) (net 4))
 (segment (start 128.27 111.76) (end 129.54 113.03) (width 0.25) (layer F.Cu) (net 4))
 (via (at 129.54 113.03) (size 0.8) (drill 0.4) (layers F.Cu B.Cu) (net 4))
 (segment (start 129.54 113.03) (end 139.7 113.03) (width 0.25) (layer B.Cu) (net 4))
 (segment (start 139.7 113.03) (end 140.97 114.3) (width 0.25) (layer B.Cu) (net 4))
 (segment (start 140.81 125.095) (end 139.065 125.095) (width 0.25) (layer F.Cu) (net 4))
 (segment (start 139.065 125.095) (end 138.43 125.73) (width 0.25) (layer F.Cu) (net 4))
 (segment (start 138.43 125.73) (end 138.43 128.27) (width 0.25) (layer F.Cu) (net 4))
 (segment (start 135.89 130.81) (end 135.4075 130.81) (width 0.25) (layer F.Cu) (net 4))
 (segment (start 138.43 128.27) (end 135.89 130.81) (width 0.25) (layer F.Cu) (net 4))
 (segment (start 135.4075 130.81) (end 137.6425 130.81) (width 0.25) (layer F.Cu) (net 4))
 (segment (start 135.89 127) (end 134.62 125.73) (width 0.25) (layer B.Cu) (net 4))
 (segment (start 144.78 120.65) (end 143.51 121.92) (width 0.25) (layer B.Cu) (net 4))
 (segment (start 134.62 125.73) (end 134.62 123.19) (width 0.25) (layer B.Cu) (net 4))
 (segment (start 142.24 127) (end 135.89 127) (width 0.25) (layer B.Cu) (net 4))
 (segment (start 146.05 120.65) (end 144.78 120.65) (width 0.25) (layer B.Cu) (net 4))
 (segment (start 143.51 121.92) (end 143.51 125.73) (width 0.25) (layer B.Cu) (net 4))
 (segment (start 143.51 125.73) (end 142.24 127) (width 0.25) (layer B.Cu) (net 4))
 (segment (start 146.05 120.65) (end 144.78 121.92) (width 0.25) (layer F.Cu) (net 4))
 (via (at 146.05 120.65) (size 1.7) (drill 1) (layers F.Cu B.Cu) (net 4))
 (segment (start 134.62 125.73) (end 134.62 129.235) (width 0.25) (layer B.Cu) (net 4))
 (segment (start 134.62 129.235) (end 134.62 130.505) (width 0.25) (layer B.Cu) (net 4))
 (segment (start 136.459989 116.930011) (end 137.16 116.23) (width 0.25) (layer B.Cu) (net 3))
 (segment (start 136.459989 121.829989) (end 136.459989 116.930011) (width 0.25) (layer B.Cu) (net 3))
 (segment (start 137.16 122.53) (end 136.459989 121.829989) (width 0.25) (layer B.Cu) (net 3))
 (segment (start 137.16 124.46) (end 138.43 125.73) (width 0.25) (layer B.Cu) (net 3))
 (segment (start 137.16 123.19) (end 137.16 124.46) (width 0.25) (layer B.Cu) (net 3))
 (segment (start 138.43 125.73) (end 140.97 125.73) (width 0.25) (layer B.Cu) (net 3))
 (segment (start 140.97 125.73) (end 142.24 124.46) (width 0.25) (layer B.Cu) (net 3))
 (segment (start 142.24 124.46) (end 142.24 120.65) (width 0.25) (layer B.Cu) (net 3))
 (segment (start 142.24 120.65) (end 144.78 118.11) (width 0.25) (layer B.Cu) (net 3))
 (segment (start 144.78 118.11) (end 146.05 118.11) (width 0.25) (layer B.Cu) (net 3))
 (segment (start 146.05 118.11) (end 146.05 118.11) (width 0.25) (layer B.Cu) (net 3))
 (via (at 146.05 118.11) (size 1.7) (drill 1) (layers F.Cu B.Cu) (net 3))
 (segment (start 147.225001 119.285001) (end 146.05 118.11) (width 0.25) (layer B.Cu) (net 3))
 (segment (start 147.225001 129.380001) (end 147.225001 119.285001) (width 0.25) (layer B.Cu) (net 3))
 (segment (start 146.100002 130.505) (end 147.225001 129.380001) (width 0.25) (layer B.Cu) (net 3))
 (segment (start 142.24 130.505) (end 146.100002 130.505) (width 0.25) (layer B.Cu) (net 3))
 (segment (start 128.27 109.7025) (end 130.81 109.7025) (width 0.25) (layer F.Cu) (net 10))
 (segment (start 130.81 109.7025) (end 130.81 109.7025) (width 0.25) (layer F.Cu) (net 10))
 (via (at 130.81 109.7025) (size 0.8) (drill 0.4) (layers F.Cu B.Cu) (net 10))
 (segment (start 128.994988 131.27999) (end 129.52749 131.27999) (width 0.25) (layer B.Cu) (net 10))
 (segment (start 127 113.5125) (end 127 129.285002) (width 0.25) (layer B.Cu) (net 10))
 (segment (start 128.524998 130.81) (end 129.235 130.81) (width 0.25) (layer B.Cu) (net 10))
 (segment (start 127 129.285002) (end 128.524998 130.81) (width 0.25) (layer B.Cu) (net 10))
 (segment (start 130.81 109.7025) (end 127 113.5125) (width 0.25) (layer B.Cu) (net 10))
 (segment (start 137.16 106.94) (end 137.16 106.04) (width 0.25) (layer F.Cu) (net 10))
 (segment (start 134.3975 109.7025) (end 137.16 106.94) (width 0.25) (layer F.Cu) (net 10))
 (segment (start 130.81 109.7025) (end 134.3975 109.7025) (width 0.25) (layer F.Cu) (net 10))
 (segment (start 136.076401 109.930009) (end 135.89 109.930009) (width 0.25) (layer F.Cu) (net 11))
 (segment (start 137.81 106.94) (end 135.89 108.86) (width 0.25) (layer F.Cu) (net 11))
 (segment (start 137.81 106.04) (end 137.81 106.94) (width 0.25) (layer F.Cu) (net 11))
 (segment (start 135.89 108.86) (end 135.89 109.79) (width 0.25) (layer F.Cu) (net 11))
 (via (at 137.16 109.7025) (size 0.8) (drill 0.4) (layers F.Cu B.Cu) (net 11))
 (segment (start 128.814999 112.485001) (end 128.814999 113.574999) (width 0.25) (layer B.Cu) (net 11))
 (segment (start 130.81 110.49) (end 128.814999 112.485001) (width 0.25) (layer B.Cu) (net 11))
 (segment (start 130.81 115.57) (end 130.81 116.20359) (width 0.25) (layer B.Cu) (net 11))
 (segment (start 128.814999 113.574999) (end 130.81 115.57) (width 0.25) (layer B.Cu) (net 11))
 (segment (start 130.084999 116.928591) (end 130.084999 118.654999) (width 0.25) (layer B.Cu) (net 11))
 (segment (start 130.81 116.20359) (end 130.084999 116.928591) (width 0.25) (layer B.Cu) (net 11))
 (segment (start 130.084999 118.654999) (end 132.08 120.65) (width 0.25) (layer B.Cu) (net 11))
 (segment (start 132.08 109.22) (end 133.35 107.95) (width 0.25) (layer B.Cu) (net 11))
 (segment (start 132.08 109.505502) (end 131.095502 110.49) (width 0.25) (layer B.Cu) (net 11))
 (segment (start 132.08 109.22) (end 132.08 109.505502) (width 0.25) (layer B.Cu) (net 11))
 (segment (start 131.095502 110.49) (end 130.81 110.49) (width 0.25) (layer B.Cu) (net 11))
 (segment (start 137.2475 109.79) (end 137.16 109.7025) (width 0.25) (layer F.Cu) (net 11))
 (segment (start 137.0725 109.79) (end 137.16 109.7025) (width 0.25) (layer F.Cu) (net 11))
 (segment (start 135.89 109.79) (end 137.0725 109.79) (width 0.25) (layer F.Cu) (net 11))
 (segment (start 135.89 107.95) (end 137.16 109.22) (width 0.25) (layer B.Cu) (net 11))
 (segment (start 135.89 107.95) (end 133.35 107.95) (width 0.25) (layer B.Cu) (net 11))
 (segment (start 137.16 109.22) (end 137.16 109.7025) (width 0.25) (layer B.Cu) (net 11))
 (segment (start 138.43 106.68) (end 138.43 106.366998) (width 0.25) (layer F.Cu) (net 12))
 (segment (start 138.46 106.04) (end 138.46 106.71) (width 0.25) (layer F.Cu) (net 12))
 (segment (start 138.46 106.71) (end 139.7 107.95) (width 0.25) (layer F.Cu) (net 12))
 (segment (start 145.16 107.95) (end 146.05 108.84) (width 0.25) (layer F.Cu) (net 12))
 (segment (start 139.7 107.95) (end 145.16 107.95) (width 0.25) (layer F.Cu) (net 12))
 (segment (start 143.51 109.7025) (end 140.97 109.7025) (width 0.25) (layer F.Cu) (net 14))
 (segment (start 140.97 109.7025) (end 139.7 109.7025) (width 0.25) (layer F.Cu) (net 14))
 (segment (start 133.285 105.84) (end 133.435 105.99) (width 0.25) (layer F.Cu) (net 8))
 (segment (start 141.035 101.665) (end 141.035 102.19) (width 0.25) (layer F.Cu) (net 8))
 (segment (start 141.035 105.84) (end 140.885 105.99) (width 0.25) (layer B.Cu) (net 8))
 (segment (start 141.035 102.19) (end 141.035 105.84) (width 0.25) (layer B.Cu) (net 8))
 (segment (start 134.41 105.99) (end 140.885 105.99) (width 0.25) (layer B.Cu) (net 8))
 (segment (start 133.435 105.99) (end 134.41 105.99) (width 0.25) (layer B.Cu) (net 8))
 (segment (start 133.285 105.84) (end 133.435 105.99) (width 0.25) (layer B.Cu) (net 8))
 (segment (start 133.285 102.19) (end 133.285 105.84) (width 0.25) (layer B.Cu) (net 8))
 (segment (start 128.27 125.73) (end 128.27 125.73) (width 0.25) (layer F.Cu) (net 15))
 (segment (start 131.445 127.635) (end 133.51 127.635) (width 0.25) (layer F.Cu) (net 15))
 (segment (start 129.54 125.73) (end 131.445 127.635) (width 0.25) (layer F.Cu) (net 15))
 (segment (start 128.27 125.73) (end 129.54 125.73) (width 0.25) (layer F.Cu) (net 15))
 (via (at 128.27 125.73) (size 1.7) (drill 1) (layers F.Cu B.Cu) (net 15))
 (segment (start 130.81 130.81) (end 130.81 127) (width 0.25) (layer B.Cu) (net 15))
 (segment (start 129.54 125.73) (end 128.27 125.73) (width 0.25) (layer B.Cu) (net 15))
 (segment (start 130.81 127) (end 129.54 125.73) (width 0.25) (layer B.Cu) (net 15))
 (segment (start 132.715 126.365) (end 133.51 126.365) (width 0.25) (layer F.Cu) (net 16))
 (segment (start 128.27 123.19) (end 128.27 123.19) (width 0.25) (layer F.Cu) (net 16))
 (segment (start 129.54 123.19) (end 132.715 126.365) (width 0.25) (layer F.Cu) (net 16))
 (segment (start 128.27 123.19) (end 129.54 123.19) (width 0.25) (layer F.Cu) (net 16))
 (via (at 128.27 123.19) (size 1.7) (drill 1) (layers F.Cu B.Cu) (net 16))
 (segment (start 129.235 122.225) (end 128.27 123.19) (width 0.25) (layer B.Cu) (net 16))
 (segment (start 132.08 122.225) (end 129.235 122.225) (width 0.25) (layer B.Cu) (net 16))
 (segment (start 133.35 124.935) (end 133.51 125.095) (width 0.25) (layer F.Cu) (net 1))
 (segment (start 133.35 121.48) (end 133.35 124.935) (width 0.25) (layer F.Cu) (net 1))
 (segment (start 136.135 123.19) (end 136.135 124.215) (width 0.25) (layer F.Cu) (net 1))
 (segment (start 135.255 125.095) (end 133.51 125.095) (width 0.25) (layer F.Cu) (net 1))
 (segment (start 136.135 124.215) (end 135.255 125.095) (width 0.25) (layer F.Cu) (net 1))
 (segment (start 129.15 120.65) (end 129.98 121.48) (width 0.25) (layer F.Cu) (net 1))
 (segment (start 128.27 120.65) (end 128.27 120.65) (width 0.25) (layer F.Cu) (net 1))
 (segment (start 133.35 121.48) (end 129.98 121.48) (width 0.25) (layer F.Cu) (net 1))
 (segment (start 128.27 120.65) (end 129.15 120.65) (width 0.25) (layer F.Cu) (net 1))
 (via (at 128.27 120.65) (size 1.7) (drill 1) (layers F.Cu B.Cu) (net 1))
 (segment (start 129.119999 115.990001) (end 136.310001 115.990001) (width 0.25) (layer F.Cu) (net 13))
 (segment (start 136.310001 115.990001) (end 138.43 118.11) (width 0.25) (layer F.Cu) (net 13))
 (segment (start 138.43 118.11) (end 140.97 118.11) (width 0.25) (layer F.Cu) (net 13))
 (segment (start 140.97 118.11) (end 142 119.14) (width 0.25) (layer F.Cu) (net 13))
 (segment (start 128.699998 115.57) (end 129.119999 115.990001) (width 0.25) (layer F.Cu) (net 13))
 (segment (start 128.27 115.57) (end 128.27 115.57) (width 0.25) (layer F.Cu) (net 13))
 (segment (start 128.27 115.57) (end 128.699998 115.57) (width 0.25) (layer F.Cu) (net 13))
 (via (at 128.27 115.57) (size 1.7) (drill 1) (layers F.Cu B.Cu) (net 13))
 (segment (start 145.415 128.905) (end 146.05 128.27) (width 0.25) (layer F.Cu) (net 7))
 (segment (start 144.145 128.905) (end 145.415 128.905) (width 0.25) (layer F.Cu) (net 7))
 (segment (start 140.81 128.905) (end 144.145 128.905) (width 0.25) (layer F.Cu) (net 7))
 (segment (start 146.05 128.27) (end 146.05 128.27) (width 0.25) (layer F.Cu) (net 7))
 (via (at 146.05 128.27) (size 1.7) (drill 1) (layers F.Cu B.Cu) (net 7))
 (segment (start 144.145 127.635) (end 146.05 125.73) (width 0.25) (layer F.Cu) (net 6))
 (segment (start 140.81 127.635) (end 144.145 127.635) (width 0.25) (layer F.Cu) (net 6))
 (segment (start 146.05 125.73) (end 146.05 125.73) (width 0.25) (layer F.Cu) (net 6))
 (via (at 146.05 125.73) (size 1.7) (drill 1) (layers F.Cu B.Cu) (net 6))
 (segment (start 146.05 123.19) (end 146.05 123.19) (width 0.25) (layer F.Cu) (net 5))
 (segment (start 140.81 126.365) (end 142.875 126.365) (width 0.25) (layer F.Cu) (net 5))
 (segment (start 146.05 123.19) (end 142.875 126.365) (width 0.25) (layer F.Cu) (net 5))
 (via (at 146.05 123.19) (size 1.7) (drill 1) (layers F.Cu B.Cu) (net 5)))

